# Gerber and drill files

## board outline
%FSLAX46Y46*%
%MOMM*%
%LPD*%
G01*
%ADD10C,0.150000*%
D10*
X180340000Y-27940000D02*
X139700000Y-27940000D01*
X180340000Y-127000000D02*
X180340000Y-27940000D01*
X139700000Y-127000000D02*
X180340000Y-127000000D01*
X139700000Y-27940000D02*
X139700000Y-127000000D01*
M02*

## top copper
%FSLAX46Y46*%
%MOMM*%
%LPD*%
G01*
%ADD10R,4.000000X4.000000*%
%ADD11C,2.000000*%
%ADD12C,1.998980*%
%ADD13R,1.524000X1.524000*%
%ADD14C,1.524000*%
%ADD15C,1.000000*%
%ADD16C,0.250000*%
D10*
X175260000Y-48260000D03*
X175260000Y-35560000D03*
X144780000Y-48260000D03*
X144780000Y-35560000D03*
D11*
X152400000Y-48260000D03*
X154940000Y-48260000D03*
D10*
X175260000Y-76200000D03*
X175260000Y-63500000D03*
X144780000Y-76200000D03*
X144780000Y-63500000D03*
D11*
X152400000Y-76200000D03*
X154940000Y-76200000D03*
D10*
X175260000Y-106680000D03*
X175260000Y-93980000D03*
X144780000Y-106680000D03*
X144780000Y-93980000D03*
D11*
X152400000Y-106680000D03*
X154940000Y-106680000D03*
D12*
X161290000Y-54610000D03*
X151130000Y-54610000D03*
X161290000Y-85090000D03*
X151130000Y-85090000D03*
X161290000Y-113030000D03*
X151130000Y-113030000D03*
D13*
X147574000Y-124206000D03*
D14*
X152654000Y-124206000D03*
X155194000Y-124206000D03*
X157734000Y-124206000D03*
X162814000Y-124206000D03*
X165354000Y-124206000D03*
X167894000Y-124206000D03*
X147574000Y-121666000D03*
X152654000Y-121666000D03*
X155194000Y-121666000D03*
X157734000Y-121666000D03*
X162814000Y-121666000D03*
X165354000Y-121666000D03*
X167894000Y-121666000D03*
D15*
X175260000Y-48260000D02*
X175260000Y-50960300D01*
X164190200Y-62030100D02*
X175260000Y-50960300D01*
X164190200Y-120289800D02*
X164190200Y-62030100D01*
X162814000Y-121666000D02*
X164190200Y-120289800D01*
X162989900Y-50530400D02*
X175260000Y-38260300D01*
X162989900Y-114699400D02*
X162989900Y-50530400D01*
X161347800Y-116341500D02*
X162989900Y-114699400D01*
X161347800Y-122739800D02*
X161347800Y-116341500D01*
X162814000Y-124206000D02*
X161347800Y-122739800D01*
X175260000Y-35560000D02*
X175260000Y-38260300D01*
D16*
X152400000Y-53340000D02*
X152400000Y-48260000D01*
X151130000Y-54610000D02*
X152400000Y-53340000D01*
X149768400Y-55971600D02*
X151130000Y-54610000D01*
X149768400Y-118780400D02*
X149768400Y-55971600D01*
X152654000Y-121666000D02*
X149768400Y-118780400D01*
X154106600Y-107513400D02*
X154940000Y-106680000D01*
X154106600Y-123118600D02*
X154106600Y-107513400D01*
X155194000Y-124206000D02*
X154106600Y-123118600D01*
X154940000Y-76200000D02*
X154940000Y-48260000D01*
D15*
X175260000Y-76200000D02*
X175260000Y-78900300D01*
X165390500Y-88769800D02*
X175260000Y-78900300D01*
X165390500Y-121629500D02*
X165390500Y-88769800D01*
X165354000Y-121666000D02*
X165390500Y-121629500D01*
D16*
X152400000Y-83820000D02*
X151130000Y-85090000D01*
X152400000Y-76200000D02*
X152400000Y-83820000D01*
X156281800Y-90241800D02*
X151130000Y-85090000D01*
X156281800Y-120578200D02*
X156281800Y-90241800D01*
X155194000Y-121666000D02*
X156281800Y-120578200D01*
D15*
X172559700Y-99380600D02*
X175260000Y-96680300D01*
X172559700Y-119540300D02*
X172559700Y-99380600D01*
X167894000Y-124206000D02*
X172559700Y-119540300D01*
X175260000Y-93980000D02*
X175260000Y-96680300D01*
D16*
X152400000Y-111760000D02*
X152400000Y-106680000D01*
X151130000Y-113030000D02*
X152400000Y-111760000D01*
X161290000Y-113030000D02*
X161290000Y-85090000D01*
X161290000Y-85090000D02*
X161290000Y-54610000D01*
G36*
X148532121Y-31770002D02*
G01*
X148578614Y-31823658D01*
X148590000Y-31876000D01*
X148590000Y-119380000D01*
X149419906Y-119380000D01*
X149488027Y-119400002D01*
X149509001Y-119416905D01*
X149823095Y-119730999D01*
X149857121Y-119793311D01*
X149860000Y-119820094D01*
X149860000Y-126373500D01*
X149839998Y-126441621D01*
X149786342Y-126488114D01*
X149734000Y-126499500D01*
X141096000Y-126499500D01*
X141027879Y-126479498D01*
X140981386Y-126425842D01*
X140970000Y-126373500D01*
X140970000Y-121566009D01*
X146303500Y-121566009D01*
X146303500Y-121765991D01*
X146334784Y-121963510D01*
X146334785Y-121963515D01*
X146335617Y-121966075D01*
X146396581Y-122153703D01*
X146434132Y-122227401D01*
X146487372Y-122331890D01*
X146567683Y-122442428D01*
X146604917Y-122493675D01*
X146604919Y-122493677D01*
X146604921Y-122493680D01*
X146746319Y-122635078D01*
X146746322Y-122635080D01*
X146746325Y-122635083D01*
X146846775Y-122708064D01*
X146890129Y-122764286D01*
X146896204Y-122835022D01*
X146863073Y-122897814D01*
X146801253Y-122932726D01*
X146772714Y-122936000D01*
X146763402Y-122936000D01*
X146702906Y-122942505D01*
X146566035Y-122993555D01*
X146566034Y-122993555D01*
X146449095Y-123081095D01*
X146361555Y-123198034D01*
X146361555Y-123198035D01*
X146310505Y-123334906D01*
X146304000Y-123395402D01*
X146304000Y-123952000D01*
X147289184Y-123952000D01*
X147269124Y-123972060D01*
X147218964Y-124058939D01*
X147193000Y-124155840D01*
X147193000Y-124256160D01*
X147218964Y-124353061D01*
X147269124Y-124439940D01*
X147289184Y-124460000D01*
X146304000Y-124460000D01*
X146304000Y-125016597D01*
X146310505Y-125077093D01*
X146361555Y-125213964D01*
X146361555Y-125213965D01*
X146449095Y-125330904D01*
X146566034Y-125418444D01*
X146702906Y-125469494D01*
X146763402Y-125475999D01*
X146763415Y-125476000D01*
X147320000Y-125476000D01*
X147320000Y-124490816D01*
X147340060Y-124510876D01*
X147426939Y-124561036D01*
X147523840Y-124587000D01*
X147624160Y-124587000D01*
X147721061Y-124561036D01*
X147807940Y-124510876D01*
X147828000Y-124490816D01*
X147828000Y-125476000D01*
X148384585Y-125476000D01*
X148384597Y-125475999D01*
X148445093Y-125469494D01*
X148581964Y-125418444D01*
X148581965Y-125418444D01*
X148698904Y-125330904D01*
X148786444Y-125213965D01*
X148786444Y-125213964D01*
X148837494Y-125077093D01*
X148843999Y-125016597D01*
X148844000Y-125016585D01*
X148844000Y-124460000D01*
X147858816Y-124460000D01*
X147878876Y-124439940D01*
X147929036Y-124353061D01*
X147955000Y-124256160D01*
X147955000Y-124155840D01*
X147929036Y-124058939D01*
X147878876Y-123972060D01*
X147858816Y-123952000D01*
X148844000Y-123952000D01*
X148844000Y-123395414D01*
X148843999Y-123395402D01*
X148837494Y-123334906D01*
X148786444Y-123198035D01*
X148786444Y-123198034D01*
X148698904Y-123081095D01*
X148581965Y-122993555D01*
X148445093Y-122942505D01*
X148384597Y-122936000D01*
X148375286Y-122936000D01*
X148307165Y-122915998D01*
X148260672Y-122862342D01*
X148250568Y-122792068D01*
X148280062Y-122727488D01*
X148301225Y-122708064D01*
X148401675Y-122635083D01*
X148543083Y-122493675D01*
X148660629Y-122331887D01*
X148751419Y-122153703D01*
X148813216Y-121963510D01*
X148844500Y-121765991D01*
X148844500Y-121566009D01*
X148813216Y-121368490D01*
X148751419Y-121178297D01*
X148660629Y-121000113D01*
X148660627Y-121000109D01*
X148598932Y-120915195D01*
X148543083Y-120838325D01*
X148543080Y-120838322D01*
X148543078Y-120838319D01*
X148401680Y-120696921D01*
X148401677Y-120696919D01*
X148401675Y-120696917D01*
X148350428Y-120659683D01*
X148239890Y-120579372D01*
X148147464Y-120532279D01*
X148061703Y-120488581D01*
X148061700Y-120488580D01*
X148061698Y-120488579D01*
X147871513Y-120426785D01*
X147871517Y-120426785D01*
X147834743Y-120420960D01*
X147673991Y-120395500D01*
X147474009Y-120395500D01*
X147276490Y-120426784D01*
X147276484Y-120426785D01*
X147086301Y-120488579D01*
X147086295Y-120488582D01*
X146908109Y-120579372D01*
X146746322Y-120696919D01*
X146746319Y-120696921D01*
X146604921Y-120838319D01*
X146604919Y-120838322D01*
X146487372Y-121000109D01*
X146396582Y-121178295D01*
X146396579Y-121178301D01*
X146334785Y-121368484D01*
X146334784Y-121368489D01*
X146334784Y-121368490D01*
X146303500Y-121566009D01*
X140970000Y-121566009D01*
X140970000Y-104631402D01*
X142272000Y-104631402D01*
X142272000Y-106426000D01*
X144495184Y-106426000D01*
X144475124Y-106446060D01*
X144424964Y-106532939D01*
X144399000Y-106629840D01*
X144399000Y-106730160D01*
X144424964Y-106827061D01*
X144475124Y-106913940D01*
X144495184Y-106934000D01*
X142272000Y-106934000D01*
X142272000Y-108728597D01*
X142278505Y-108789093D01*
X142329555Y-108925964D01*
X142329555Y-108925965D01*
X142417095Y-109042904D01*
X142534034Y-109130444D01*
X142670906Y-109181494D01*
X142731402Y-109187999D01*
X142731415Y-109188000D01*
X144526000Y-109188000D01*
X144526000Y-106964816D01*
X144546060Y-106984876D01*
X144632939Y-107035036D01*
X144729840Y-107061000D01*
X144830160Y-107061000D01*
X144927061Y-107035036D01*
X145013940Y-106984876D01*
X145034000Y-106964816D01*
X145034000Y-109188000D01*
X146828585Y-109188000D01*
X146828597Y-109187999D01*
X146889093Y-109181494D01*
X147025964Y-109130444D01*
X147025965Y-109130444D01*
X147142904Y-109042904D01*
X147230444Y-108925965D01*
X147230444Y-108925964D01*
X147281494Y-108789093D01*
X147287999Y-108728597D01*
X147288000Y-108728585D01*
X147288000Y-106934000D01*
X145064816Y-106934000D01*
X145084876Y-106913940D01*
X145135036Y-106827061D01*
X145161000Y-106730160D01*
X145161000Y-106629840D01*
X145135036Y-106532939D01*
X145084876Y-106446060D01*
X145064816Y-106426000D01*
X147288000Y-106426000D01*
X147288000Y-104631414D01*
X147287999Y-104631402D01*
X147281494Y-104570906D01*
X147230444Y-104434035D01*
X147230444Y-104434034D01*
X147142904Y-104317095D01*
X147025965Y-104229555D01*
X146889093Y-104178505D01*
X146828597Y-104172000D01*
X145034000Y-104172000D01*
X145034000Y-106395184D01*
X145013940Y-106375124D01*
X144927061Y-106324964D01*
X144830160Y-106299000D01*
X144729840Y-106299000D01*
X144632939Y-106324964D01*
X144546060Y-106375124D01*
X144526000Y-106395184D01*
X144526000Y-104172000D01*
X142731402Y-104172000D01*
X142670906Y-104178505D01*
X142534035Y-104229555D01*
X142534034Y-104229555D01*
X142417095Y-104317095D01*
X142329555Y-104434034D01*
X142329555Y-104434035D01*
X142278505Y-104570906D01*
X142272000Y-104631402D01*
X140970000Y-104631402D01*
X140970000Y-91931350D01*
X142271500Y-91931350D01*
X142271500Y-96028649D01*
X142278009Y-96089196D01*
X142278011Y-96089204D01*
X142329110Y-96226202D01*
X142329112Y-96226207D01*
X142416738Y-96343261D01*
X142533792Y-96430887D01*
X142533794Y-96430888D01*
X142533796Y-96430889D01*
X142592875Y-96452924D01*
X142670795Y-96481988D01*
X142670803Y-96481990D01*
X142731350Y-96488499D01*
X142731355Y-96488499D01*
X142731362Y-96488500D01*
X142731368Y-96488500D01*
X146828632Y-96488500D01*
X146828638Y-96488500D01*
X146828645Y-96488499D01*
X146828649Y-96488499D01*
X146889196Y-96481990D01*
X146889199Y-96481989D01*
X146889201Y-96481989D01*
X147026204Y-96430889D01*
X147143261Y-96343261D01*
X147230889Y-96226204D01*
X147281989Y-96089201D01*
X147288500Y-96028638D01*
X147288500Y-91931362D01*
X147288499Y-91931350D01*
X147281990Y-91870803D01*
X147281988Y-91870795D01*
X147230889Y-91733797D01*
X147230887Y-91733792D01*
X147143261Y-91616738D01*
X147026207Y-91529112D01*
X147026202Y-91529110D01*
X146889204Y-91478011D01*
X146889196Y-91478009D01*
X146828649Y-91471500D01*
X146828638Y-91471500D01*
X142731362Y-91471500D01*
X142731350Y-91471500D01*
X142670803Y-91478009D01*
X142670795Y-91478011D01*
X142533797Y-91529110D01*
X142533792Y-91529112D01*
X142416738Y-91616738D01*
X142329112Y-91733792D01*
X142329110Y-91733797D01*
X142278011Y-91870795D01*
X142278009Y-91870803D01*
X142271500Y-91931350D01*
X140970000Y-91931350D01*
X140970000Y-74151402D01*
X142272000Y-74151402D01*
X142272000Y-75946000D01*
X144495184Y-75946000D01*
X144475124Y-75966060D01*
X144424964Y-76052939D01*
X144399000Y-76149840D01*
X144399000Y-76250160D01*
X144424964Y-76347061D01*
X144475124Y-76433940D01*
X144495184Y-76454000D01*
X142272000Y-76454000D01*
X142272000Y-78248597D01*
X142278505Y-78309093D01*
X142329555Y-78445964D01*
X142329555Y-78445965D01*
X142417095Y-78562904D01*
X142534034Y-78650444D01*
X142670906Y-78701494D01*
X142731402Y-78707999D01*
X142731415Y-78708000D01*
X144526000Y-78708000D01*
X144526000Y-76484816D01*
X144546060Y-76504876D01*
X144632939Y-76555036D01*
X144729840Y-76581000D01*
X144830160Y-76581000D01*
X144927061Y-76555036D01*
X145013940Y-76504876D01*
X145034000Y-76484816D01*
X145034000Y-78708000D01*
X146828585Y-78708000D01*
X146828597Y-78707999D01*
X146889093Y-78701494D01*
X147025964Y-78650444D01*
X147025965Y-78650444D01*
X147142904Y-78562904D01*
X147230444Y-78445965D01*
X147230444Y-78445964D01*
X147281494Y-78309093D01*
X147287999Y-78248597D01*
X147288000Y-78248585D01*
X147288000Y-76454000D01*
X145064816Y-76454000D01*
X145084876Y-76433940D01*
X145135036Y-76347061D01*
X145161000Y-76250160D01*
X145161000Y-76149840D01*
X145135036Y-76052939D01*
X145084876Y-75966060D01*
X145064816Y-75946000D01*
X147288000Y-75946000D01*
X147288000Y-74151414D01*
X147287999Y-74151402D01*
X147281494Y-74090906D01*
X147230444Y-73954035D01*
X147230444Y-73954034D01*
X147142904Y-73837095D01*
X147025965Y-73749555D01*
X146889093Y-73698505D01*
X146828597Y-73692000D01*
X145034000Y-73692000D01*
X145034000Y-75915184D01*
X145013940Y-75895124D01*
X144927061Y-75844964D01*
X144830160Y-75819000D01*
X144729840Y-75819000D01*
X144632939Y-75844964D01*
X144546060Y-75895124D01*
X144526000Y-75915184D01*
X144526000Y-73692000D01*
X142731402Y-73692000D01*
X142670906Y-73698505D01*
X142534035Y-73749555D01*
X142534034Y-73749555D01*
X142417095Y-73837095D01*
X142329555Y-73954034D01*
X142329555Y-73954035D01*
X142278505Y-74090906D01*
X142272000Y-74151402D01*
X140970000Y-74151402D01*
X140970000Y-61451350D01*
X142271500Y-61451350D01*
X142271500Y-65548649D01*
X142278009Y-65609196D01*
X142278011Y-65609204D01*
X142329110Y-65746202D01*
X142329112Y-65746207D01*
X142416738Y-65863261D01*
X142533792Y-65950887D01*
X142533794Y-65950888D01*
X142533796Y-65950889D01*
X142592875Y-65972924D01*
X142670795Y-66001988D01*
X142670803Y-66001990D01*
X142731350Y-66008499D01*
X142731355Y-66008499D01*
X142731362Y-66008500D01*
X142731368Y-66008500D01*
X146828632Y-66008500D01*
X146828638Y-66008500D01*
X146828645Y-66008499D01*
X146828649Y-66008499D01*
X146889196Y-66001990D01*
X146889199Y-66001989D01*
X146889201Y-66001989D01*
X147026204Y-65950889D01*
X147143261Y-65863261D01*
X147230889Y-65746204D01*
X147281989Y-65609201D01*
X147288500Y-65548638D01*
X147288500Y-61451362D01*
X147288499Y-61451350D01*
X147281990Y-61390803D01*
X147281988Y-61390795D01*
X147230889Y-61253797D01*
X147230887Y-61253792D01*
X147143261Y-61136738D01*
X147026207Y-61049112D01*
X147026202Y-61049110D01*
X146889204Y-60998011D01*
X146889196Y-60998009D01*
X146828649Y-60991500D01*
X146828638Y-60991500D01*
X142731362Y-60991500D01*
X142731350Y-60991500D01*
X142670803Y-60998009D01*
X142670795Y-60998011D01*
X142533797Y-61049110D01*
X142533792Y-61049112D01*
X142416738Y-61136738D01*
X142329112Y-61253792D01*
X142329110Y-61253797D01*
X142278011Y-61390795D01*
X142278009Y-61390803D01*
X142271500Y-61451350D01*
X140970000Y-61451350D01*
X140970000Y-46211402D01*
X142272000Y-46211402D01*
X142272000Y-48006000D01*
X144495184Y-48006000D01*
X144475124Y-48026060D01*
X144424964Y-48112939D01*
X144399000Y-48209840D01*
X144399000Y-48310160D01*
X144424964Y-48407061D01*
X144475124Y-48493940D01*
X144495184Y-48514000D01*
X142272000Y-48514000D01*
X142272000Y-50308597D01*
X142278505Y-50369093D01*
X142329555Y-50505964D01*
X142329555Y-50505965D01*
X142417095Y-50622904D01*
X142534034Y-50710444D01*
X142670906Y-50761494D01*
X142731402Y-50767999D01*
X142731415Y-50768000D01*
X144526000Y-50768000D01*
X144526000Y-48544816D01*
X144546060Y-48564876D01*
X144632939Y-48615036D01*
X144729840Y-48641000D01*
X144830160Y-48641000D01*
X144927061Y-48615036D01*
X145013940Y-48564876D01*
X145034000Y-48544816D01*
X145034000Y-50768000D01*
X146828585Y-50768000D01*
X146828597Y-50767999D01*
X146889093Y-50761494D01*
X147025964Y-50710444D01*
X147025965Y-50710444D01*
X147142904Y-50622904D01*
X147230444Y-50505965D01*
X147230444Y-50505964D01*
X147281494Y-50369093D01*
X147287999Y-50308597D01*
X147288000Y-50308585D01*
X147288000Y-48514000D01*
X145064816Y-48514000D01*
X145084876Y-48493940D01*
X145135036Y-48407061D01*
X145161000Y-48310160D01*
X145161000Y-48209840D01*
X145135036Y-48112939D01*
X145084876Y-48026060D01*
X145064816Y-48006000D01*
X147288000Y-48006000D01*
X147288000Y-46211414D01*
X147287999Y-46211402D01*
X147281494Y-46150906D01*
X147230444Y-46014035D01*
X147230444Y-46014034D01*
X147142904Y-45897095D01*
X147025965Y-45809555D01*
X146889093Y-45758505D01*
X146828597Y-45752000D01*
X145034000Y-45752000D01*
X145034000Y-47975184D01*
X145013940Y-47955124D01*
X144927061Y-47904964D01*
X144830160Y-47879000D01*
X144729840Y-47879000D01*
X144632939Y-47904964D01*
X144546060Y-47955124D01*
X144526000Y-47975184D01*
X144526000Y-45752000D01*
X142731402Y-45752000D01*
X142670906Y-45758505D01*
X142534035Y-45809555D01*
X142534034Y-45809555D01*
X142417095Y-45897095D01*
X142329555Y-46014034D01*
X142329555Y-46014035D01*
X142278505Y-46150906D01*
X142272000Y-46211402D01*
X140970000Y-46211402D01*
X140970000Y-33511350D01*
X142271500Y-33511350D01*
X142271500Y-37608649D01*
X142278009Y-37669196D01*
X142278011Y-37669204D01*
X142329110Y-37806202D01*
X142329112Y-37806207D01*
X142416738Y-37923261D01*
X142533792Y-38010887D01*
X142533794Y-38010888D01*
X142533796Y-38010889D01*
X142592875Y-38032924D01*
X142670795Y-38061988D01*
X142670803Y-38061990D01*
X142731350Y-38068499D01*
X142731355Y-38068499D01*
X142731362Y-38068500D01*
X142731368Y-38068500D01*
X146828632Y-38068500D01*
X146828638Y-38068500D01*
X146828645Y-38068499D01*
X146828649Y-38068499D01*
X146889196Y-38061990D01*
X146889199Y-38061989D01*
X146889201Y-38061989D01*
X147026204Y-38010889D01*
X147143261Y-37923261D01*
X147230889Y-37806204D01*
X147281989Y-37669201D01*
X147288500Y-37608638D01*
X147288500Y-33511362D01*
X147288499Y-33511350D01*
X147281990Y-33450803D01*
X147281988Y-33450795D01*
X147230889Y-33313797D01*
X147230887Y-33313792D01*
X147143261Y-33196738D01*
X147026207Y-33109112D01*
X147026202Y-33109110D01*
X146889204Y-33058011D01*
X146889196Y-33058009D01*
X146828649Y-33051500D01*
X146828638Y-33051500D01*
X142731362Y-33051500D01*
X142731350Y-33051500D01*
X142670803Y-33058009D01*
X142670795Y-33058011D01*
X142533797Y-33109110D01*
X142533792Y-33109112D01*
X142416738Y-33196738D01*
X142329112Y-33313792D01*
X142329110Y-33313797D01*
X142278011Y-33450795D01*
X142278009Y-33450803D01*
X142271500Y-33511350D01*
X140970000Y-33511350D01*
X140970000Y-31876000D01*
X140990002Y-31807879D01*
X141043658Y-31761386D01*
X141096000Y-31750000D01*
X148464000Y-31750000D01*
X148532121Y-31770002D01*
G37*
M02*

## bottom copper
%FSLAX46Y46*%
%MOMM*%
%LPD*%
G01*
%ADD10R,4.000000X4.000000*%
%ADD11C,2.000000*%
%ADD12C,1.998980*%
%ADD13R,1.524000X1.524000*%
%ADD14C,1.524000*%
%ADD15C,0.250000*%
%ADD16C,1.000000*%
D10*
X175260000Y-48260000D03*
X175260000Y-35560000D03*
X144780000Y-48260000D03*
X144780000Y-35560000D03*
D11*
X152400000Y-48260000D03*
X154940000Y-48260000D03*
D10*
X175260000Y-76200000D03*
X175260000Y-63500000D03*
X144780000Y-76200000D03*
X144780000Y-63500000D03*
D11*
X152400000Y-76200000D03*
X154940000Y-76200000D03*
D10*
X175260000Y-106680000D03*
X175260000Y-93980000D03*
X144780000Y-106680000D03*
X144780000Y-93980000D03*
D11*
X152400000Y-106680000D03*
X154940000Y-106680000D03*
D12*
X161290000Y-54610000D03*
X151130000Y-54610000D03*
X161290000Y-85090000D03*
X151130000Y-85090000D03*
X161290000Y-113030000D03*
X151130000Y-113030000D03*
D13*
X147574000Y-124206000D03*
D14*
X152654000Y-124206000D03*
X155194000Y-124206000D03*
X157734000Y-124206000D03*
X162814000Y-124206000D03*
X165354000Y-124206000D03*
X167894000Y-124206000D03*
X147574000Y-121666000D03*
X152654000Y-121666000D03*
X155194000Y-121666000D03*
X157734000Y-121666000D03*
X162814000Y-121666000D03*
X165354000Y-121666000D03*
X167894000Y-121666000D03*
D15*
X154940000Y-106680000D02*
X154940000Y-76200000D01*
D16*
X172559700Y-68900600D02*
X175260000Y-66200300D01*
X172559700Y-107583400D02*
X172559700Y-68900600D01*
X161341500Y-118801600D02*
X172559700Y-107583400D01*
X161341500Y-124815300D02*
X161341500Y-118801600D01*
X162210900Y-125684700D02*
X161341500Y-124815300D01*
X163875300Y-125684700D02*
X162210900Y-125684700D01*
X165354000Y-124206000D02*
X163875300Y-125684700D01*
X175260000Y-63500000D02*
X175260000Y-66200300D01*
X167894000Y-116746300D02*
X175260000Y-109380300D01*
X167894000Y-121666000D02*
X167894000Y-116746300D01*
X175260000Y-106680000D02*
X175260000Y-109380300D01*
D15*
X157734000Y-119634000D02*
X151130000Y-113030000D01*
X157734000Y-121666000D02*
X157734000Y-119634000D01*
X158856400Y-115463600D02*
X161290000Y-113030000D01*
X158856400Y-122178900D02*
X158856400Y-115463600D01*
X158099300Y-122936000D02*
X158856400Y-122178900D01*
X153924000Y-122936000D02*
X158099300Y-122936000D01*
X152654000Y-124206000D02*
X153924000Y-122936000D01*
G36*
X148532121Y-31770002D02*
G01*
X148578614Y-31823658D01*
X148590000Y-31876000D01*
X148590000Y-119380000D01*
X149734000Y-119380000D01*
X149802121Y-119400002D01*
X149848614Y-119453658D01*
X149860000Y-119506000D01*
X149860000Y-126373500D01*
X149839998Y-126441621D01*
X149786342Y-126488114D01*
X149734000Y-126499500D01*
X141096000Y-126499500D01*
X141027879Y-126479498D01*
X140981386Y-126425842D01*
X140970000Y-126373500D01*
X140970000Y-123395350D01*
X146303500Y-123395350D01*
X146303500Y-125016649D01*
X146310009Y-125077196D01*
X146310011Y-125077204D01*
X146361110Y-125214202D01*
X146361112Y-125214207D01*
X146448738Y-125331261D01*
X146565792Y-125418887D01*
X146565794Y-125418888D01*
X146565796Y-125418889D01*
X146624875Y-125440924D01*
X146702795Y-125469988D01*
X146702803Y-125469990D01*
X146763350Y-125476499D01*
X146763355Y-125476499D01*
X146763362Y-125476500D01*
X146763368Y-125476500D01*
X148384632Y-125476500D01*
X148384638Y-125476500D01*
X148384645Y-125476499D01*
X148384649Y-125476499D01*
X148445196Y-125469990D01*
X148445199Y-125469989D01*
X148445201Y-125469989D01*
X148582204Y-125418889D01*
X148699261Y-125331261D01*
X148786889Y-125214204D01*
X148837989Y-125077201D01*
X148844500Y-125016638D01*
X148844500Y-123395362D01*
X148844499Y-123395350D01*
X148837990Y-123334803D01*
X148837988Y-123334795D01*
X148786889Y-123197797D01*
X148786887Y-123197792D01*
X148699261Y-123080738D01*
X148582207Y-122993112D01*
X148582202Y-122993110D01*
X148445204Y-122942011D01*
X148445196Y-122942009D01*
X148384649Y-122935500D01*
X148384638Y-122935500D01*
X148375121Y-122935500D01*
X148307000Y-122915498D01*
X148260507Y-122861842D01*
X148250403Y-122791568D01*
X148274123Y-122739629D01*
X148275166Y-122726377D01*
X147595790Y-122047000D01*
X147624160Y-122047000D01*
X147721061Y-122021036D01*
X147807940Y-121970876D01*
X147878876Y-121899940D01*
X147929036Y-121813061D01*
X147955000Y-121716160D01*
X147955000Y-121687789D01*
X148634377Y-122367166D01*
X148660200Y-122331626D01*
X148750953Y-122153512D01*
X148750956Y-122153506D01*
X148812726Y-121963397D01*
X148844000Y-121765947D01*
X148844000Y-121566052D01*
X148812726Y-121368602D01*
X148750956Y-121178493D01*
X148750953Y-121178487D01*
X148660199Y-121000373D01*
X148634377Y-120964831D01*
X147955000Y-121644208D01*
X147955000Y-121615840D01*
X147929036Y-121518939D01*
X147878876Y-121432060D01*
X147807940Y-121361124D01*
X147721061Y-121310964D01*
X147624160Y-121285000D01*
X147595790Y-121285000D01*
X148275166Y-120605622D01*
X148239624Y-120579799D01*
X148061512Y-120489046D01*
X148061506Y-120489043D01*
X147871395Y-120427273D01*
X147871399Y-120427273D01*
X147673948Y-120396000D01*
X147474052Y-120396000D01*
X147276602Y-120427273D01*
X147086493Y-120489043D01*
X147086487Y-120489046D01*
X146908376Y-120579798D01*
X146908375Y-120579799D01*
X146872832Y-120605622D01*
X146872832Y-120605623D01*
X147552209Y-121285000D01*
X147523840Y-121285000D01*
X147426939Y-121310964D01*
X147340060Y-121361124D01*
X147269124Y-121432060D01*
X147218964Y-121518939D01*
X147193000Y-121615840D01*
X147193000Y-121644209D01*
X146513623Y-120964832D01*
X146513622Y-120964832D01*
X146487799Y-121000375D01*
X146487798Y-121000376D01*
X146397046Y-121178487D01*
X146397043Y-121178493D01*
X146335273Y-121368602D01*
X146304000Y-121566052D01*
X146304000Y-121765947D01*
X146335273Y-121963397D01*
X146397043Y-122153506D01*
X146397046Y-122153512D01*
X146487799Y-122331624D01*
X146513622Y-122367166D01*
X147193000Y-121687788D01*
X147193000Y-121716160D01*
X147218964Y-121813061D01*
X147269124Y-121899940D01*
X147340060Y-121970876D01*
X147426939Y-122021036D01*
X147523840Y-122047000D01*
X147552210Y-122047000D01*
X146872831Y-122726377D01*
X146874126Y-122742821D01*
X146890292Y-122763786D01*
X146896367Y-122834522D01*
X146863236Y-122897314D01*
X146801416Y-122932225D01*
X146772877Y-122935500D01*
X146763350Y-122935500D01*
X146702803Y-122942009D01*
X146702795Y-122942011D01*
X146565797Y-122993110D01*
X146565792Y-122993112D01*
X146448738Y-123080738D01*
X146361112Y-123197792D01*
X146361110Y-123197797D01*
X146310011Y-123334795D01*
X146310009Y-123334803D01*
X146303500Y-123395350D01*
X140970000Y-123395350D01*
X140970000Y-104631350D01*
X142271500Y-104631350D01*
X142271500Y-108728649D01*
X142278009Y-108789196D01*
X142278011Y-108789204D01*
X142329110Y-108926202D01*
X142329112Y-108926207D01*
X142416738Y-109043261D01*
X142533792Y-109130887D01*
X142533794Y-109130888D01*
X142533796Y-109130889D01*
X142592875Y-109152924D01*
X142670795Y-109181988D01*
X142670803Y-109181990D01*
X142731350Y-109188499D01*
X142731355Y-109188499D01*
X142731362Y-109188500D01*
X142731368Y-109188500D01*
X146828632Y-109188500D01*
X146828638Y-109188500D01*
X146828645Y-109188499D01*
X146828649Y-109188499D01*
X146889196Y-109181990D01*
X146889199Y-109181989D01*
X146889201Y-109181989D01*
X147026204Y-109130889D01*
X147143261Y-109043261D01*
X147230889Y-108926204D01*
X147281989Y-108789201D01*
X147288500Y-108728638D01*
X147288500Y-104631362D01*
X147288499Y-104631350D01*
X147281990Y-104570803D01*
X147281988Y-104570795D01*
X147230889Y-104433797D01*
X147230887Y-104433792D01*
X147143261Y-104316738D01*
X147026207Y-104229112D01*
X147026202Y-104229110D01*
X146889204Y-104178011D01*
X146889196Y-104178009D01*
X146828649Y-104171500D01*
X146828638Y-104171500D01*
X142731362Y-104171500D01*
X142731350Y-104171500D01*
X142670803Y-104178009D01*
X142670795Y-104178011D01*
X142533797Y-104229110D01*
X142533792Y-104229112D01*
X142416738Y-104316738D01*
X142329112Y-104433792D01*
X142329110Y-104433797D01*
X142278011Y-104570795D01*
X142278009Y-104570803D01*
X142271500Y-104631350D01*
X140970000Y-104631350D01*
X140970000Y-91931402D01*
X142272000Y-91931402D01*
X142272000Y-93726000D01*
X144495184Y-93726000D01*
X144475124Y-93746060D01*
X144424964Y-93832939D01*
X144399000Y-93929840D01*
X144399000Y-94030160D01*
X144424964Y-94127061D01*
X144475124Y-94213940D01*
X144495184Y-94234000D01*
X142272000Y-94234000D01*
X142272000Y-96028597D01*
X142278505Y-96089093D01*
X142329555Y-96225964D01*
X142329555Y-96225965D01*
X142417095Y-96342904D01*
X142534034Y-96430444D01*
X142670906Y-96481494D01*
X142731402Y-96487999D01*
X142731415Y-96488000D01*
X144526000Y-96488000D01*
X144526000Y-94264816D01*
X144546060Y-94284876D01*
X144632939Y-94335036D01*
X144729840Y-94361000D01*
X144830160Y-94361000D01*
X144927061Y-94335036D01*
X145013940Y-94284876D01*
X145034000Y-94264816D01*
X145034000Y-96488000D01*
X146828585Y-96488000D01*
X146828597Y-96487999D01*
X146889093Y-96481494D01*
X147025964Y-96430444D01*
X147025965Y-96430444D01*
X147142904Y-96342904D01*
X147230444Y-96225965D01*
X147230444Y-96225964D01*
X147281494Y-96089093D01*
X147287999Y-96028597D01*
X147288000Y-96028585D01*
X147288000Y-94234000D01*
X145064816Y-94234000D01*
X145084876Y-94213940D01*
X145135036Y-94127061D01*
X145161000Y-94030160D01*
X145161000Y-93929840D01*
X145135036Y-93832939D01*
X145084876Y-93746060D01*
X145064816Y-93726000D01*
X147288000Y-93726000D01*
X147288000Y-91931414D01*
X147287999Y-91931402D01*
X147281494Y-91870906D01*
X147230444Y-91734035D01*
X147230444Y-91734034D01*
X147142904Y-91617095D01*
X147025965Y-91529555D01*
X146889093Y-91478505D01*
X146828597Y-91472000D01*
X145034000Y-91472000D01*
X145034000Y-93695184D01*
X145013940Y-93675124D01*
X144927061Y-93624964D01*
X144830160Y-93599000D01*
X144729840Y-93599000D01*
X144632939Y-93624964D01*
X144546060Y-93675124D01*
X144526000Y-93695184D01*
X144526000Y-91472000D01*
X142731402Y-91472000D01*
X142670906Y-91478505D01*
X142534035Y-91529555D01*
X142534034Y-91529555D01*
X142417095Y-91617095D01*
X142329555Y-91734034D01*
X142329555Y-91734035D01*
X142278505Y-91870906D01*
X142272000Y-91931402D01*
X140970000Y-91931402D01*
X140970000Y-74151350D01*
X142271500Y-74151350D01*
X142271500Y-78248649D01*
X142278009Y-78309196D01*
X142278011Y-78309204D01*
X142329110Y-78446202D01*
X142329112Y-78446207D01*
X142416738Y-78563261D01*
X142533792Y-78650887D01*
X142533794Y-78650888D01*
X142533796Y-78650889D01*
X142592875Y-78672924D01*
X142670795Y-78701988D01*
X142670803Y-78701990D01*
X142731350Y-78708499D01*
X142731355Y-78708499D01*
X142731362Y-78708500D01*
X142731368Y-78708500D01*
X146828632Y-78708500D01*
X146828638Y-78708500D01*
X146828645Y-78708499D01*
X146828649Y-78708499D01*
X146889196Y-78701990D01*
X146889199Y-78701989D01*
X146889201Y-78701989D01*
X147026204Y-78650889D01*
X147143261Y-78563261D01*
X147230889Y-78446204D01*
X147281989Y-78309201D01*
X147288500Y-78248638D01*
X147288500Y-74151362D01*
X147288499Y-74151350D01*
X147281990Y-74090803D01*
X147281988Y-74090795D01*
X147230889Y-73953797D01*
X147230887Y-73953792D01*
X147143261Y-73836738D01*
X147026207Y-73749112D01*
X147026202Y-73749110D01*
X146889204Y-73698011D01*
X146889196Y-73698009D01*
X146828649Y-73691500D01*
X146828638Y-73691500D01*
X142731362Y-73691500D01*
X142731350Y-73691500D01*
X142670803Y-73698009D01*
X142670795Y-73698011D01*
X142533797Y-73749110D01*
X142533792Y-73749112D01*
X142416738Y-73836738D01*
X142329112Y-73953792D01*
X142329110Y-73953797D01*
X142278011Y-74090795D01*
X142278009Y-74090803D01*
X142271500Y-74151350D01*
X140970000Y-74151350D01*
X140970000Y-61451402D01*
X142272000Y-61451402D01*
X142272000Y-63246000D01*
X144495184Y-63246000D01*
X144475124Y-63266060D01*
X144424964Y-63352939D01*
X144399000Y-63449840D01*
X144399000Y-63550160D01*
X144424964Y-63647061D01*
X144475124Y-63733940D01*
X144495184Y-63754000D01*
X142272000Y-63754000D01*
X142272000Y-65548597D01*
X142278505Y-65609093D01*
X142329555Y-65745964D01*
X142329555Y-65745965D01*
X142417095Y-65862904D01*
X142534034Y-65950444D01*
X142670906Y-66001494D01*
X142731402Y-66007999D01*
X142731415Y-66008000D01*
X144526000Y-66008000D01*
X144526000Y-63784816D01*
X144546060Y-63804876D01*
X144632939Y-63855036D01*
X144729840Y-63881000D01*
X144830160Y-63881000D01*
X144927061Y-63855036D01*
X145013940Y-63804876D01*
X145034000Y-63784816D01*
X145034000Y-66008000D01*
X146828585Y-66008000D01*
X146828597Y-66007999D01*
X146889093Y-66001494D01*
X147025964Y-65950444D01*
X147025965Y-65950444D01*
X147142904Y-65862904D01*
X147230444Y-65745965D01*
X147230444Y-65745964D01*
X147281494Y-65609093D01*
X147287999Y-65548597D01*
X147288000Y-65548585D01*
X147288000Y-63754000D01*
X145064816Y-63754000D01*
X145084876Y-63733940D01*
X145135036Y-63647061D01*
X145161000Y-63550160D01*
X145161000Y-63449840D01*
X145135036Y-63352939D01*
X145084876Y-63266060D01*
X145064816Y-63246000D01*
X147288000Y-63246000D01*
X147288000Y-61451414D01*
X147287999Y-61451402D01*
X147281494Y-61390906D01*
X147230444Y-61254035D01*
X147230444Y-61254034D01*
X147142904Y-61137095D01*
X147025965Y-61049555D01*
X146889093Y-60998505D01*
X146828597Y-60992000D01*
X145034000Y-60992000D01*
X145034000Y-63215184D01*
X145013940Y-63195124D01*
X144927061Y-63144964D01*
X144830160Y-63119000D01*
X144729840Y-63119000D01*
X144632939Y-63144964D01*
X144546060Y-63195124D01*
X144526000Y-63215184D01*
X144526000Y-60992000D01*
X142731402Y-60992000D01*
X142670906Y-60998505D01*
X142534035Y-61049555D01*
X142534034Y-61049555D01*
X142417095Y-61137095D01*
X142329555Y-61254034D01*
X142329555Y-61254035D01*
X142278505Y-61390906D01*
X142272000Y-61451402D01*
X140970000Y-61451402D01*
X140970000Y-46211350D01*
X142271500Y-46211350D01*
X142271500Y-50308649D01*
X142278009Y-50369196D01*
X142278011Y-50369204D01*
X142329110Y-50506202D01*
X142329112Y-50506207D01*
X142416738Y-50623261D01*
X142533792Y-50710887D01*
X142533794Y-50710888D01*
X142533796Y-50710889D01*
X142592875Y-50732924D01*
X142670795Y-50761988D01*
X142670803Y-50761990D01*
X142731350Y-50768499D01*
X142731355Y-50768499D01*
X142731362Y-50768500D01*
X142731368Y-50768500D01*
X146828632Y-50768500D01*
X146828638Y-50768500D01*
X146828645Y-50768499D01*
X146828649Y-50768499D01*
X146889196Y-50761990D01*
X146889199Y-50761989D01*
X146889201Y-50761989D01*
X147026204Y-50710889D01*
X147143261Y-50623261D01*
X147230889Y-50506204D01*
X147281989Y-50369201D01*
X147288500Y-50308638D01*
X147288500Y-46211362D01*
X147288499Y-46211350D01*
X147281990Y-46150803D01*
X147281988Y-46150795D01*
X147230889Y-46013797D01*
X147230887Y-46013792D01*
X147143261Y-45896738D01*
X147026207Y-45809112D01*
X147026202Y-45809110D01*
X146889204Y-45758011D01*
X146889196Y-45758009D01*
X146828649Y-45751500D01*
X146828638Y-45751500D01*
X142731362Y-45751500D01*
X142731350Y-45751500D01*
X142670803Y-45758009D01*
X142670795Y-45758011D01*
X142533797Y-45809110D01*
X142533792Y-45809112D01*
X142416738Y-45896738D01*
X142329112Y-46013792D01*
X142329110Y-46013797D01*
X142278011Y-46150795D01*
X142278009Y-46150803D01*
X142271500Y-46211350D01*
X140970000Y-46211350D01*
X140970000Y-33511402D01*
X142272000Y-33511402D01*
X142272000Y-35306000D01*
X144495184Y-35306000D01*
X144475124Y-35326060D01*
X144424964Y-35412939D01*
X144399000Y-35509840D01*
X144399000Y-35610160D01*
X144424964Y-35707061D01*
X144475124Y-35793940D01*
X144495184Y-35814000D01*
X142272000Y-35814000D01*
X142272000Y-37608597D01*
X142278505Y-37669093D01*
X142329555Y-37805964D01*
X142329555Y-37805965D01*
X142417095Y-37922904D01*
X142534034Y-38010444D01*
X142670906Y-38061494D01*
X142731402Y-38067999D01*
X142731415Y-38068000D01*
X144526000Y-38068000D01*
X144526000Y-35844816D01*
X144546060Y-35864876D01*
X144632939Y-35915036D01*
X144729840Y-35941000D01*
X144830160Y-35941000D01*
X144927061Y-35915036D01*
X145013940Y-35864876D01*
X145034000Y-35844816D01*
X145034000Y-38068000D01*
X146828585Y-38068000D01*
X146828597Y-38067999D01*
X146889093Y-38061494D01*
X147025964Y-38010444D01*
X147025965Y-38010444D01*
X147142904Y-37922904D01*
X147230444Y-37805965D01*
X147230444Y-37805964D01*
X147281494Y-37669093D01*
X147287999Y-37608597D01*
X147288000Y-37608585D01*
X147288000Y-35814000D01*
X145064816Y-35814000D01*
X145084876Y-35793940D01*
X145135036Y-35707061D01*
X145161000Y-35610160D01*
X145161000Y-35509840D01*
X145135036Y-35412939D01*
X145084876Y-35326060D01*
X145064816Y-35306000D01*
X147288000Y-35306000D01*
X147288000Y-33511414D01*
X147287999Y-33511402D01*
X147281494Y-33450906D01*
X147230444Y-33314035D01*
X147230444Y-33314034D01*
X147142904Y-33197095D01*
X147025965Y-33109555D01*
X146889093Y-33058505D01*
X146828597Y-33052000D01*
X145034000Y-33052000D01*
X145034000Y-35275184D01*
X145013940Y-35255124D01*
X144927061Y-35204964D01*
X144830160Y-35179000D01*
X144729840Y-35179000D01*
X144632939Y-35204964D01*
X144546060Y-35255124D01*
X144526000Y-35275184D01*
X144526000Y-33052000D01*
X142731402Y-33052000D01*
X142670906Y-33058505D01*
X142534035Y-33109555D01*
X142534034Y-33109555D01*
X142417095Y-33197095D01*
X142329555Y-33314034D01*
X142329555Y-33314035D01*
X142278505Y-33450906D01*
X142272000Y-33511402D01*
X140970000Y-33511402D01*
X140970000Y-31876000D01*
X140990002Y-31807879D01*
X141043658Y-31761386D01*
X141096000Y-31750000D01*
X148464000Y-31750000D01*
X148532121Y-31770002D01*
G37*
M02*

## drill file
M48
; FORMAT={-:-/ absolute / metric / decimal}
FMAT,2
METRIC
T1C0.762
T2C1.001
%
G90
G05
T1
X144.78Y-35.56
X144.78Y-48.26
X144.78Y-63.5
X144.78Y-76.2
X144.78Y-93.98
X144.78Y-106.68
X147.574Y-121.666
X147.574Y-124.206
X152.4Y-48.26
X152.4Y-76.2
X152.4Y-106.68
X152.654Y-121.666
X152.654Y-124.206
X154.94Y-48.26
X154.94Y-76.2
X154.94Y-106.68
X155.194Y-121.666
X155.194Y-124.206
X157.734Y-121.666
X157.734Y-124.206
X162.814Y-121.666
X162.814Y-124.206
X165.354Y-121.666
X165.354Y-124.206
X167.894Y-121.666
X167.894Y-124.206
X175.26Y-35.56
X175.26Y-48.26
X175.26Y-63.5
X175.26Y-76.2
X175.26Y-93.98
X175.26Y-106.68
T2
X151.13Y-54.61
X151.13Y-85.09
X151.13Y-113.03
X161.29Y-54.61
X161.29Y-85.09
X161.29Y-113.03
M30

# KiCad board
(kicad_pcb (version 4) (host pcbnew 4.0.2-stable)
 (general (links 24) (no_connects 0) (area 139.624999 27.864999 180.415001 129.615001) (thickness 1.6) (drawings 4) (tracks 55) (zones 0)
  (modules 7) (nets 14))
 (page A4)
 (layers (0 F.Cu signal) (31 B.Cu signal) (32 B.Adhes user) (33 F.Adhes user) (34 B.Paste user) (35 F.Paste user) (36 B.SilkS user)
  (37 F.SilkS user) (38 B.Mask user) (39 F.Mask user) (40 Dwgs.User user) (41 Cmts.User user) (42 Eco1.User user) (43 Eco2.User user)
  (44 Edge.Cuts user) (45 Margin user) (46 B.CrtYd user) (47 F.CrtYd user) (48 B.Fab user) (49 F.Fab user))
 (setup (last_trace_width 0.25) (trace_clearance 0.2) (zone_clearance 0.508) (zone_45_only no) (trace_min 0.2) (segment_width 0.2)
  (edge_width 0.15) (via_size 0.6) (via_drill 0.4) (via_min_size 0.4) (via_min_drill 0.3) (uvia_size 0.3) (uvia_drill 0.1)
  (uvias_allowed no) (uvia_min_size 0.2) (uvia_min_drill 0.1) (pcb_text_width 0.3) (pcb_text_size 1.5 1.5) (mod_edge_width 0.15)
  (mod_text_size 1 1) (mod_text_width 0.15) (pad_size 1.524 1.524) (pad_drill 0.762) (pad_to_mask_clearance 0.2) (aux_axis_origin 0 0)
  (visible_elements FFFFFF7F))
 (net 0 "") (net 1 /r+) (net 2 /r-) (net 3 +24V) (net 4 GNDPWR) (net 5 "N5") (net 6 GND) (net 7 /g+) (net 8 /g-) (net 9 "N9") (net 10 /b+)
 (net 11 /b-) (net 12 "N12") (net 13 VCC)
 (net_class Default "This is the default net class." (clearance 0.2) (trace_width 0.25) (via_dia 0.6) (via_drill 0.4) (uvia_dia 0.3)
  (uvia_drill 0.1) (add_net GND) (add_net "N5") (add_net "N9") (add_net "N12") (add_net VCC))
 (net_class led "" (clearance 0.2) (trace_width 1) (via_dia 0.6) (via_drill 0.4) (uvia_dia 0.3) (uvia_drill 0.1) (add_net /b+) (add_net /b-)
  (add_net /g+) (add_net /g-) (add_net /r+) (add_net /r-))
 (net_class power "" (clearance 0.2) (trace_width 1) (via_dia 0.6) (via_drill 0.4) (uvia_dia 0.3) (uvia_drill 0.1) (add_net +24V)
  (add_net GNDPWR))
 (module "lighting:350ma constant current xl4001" (layer F.Cu) (at 175.26 48.26 90)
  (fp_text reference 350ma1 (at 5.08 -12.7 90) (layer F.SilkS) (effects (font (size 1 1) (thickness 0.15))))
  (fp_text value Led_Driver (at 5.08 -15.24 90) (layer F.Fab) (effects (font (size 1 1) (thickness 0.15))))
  (pad 3 thru_hole rect (at 0 0 90) (size 4 4) (drill 0.762) (layers *.Cu *.Mask F.SilkS) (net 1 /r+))
  (pad 4 thru_hole rect (at 12.7 0 90) (size 4 4) (drill 0.762) (layers *.Cu *.Mask F.SilkS) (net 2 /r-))
  (pad 1 thru_hole rect (at 0 -30.48 90) (size 4 4) (drill 0.762) (layers *.Cu *.Mask F.SilkS) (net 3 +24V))
  (pad 2 thru_hole rect (at 12.7 -30.48 90) (size 4 4) (drill 0.762) (layers *.Cu *.Mask F.SilkS) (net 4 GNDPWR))
  (pad 5 thru_hole circle (at 0 -22.86 90) (size 2 2) (drill 0.762) (layers *.Cu *.Mask F.SilkS) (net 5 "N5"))
  (pad 6 thru_hole circle (at 0 -20.32 90) (size 2 2) (drill 0.762) (layers *.Cu *.Mask F.SilkS) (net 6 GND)))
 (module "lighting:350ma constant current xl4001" (layer F.Cu) (at 175.26 76.2 90)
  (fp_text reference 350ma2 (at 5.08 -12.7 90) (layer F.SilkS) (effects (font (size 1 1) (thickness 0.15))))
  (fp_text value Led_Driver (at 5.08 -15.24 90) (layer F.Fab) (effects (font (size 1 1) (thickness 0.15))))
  (pad 3 thru_hole rect (at 0 0 90) (size 4 4) (drill 0.762) (layers *.Cu *.Mask F.SilkS) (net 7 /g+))
  (pad 4 thru_hole rect (at 12.7 0 90) (size 4 4) (drill 0.762) (layers *.Cu *.Mask F.SilkS) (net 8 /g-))
  (pad 1 thru_hole rect (at 0 -30.48 90) (size 4 4) (drill 0.762) (layers *.Cu *.Mask F.SilkS) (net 3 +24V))
  (pad 2 thru_hole rect (at 12.7 -30.48 90) (size 4 4) (drill 0.762) (layers *.Cu *.Mask F.SilkS) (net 4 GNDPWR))
  (pad 5 thru_hole circle (at 0 -22.86 90) (size 2 2) (drill 0.762) (layers *.Cu *.Mask F.SilkS) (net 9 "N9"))
  (pad 6 thru_hole circle (at 0 -20.32 90) (size 2 2) (drill 0.762) (layers *.Cu *.Mask F.SilkS) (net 6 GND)))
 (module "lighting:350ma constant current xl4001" (layer F.Cu) (at 175.26 106.68 90)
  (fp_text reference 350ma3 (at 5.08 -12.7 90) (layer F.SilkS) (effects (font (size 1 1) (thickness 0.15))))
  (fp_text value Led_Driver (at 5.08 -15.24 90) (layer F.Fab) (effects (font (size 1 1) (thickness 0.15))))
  (pad 3 thru_hole rect (at 0 0 90) (size 4 4) (drill 0.762) (layers *.Cu *.Mask F.SilkS) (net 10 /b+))
  (pad 4 thru_hole rect (at 12.7 0 90) (size 4 4) (drill 0.762) (layers *.Cu *.Mask F.SilkS) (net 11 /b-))
  (pad 1 thru_hole rect (at 0 -30.48 90) (size 4 4) (drill 0.762) (layers *.Cu *.Mask F.SilkS) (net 3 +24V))
  (pad 2 thru_hole rect (at 12.7 -30.48 90) (size 4 4) (drill 0.762) (layers *.Cu *.Mask F.SilkS) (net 4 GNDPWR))
  (pad 5 thru_hole circle (at 0 -22.86 90) (size 2 2) (drill 0.762) (layers *.Cu *.Mask F.SilkS) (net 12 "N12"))
  (pad 6 thru_hole circle (at 0 -20.32 90) (size 2 2) (drill 0.762) (layers *.Cu *.Mask F.SilkS) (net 6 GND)))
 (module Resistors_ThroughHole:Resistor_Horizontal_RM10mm (layer F.Cu) (at 161.29 54.61 180)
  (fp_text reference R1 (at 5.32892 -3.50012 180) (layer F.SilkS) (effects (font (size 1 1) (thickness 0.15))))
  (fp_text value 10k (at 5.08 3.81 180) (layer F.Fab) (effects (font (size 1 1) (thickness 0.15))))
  (pad 1 thru_hole circle (at 0 0 180) (size 1.99898 1.99898) (drill 1.00076) (layers *.Cu *.SilkS *.Mask) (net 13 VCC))
  (pad 2 thru_hole circle (at 10.16 0 180) (size 1.99898 1.99898) (drill 1.00076) (layers *.Cu *.SilkS *.Mask) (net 5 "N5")))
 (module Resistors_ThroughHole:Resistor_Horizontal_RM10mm (layer F.Cu) (at 161.29 85.09 180)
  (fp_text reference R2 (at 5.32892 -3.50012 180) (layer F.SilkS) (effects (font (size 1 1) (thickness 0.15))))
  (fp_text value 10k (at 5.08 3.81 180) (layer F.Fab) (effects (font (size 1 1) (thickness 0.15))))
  (pad 1 thru_hole circle (at 0 0 180) (size 1.99898 1.99898) (drill 1.00076) (layers *.Cu *.SilkS *.Mask) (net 13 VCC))
  (pad 2 thru_hole circle (at 10.16 0 180) (size 1.99898 1.99898) (drill 1.00076) (layers *.Cu *.SilkS *.Mask) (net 9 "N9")))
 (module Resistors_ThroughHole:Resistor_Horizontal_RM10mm (layer F.Cu) (at 161.29 113.03 180)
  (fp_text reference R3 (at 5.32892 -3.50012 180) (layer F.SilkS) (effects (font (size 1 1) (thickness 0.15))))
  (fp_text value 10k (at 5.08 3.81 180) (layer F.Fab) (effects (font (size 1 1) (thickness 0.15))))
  (pad 1 thru_hole circle (at 0 0 180) (size 1.99898 1.99898) (drill 1.00076) (layers *.Cu *.SilkS *.Mask) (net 13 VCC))
  (pad 2 thru_hole circle (at 10.16 0 180) (size 1.99898 1.99898) (drill 1.00076) (layers *.Cu *.SilkS *.Mask) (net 12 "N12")))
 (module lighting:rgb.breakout (layer F.Cu) (at 150.114 124.206)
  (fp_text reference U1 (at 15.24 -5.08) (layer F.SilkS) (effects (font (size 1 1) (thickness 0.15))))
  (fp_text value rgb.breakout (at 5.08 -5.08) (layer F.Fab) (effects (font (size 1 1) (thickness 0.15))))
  (pad 1 thru_hole rect (at -2.54 0) (size 1.524 1.524) (drill 0.762) (layers *.Cu *.Mask F.SilkS) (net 3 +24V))
  (pad 3 thru_hole circle (at 2.54 0) (size 1.524 1.524) (drill 0.762) (layers *.Cu *.Mask F.SilkS) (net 13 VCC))
  (pad 4 thru_hole circle (at 5.08 0) (size 1.524 1.524) (drill 0.762) (layers *.Cu *.Mask F.SilkS) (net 6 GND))
  (pad "" thru_hole circle (at 7.62 0) (size 1.524 1.524) (drill 0.762) (layers *.Cu *.Mask F.SilkS))
  (pad 9 thru_hole circle (at 12.7 0) (size 1.524 1.524) (drill 0.762) (layers *.Cu *.Mask F.SilkS) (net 2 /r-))
  (pad 11 thru_hole circle (at 15.24 0) (size 1.524 1.524) (drill 0.762) (layers *.Cu *.Mask F.SilkS) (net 8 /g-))
  (pad 13 thru_hole circle (at 17.78 0) (size 1.524 1.524) (drill 0.762) (layers *.Cu *.Mask F.SilkS) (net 11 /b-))
  (pad 2 thru_hole circle (at -2.54 -2.54) (size 1.524 1.524) (drill 0.762) (layers *.Cu *.Mask F.SilkS) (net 4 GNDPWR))
  (pad 5 thru_hole circle (at 2.54 -2.54) (size 1.524 1.524) (drill 0.762) (layers *.Cu *.Mask F.SilkS) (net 5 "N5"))
  (pad 6 thru_hole circle (at 5.08 -2.54) (size 1.524 1.524) (drill 0.762) (layers *.Cu *.Mask F.SilkS) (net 9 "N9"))
  (pad 7 thru_hole circle (at 7.62 -2.54) (size 1.524 1.524) (drill 0.762) (layers *.Cu *.Mask F.SilkS) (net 12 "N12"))
  (pad 8 thru_hole circle (at 12.7 -2.54) (size 1.524 1.524) (drill 0.762) (layers *.Cu *.Mask F.SilkS) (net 1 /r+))
  (pad 10 thru_hole circle (at 15.24 -2.54) (size 1.524 1.524) (drill 0.762) (layers *.Cu *.Mask F.SilkS) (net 7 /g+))
  (pad 12 thru_hole circle (at 17.78 -2.54) (size 1.524 1.524) (drill 0.762) (layers *.Cu *.Mask F.SilkS) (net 10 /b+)))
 (gr_line (start 180.34 27.94) (end 139.7 27.94) (angle 90) (layer Edge.Cuts) (width 0.15))
 (gr_line (start 180.34 127) (end 180.34 27.94) (angle 90) (layer Edge.Cuts) (width 0.15))
 (gr_line (start 139.7 127) (end 180.34 127) (angle 90) (layer Edge.Cuts) (width 0.15))
 (gr_line (start 139.7 27.94) (end 139.7 127) (angle 90) (layer Edge.Cuts) (width 0.15))
 (segment (start 175.26 48.26) (end 175.26 50.9603) (width 1) (layer F.Cu) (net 1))
 (segment (start 164.1902 62.0301) (end 175.26 50.9603) (width 1) (layer F.Cu) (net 1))
 (segment (start 164.1902 120.2898) (end 164.1902 62.0301) (width 1) (layer F.Cu) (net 1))
 (segment (start 162.814 121.666) (end 164.1902 120.2898) (width 1) (layer F.Cu) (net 1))
 (segment (start 162.9899 50.5304) (end 175.26 38.2603) (width 1) (layer F.Cu) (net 2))
 (segment (start 162.9899 114.6994) (end 162.9899 50.5304) (width 1) (layer F.Cu) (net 2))
 (segment (start 161.3478 116.3415) (end 162.9899 114.6994) (width 1) (layer F.Cu) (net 2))
 (segment (start 161.3478 122.7398) (end 161.3478 116.3415) (width 1) (layer F.Cu) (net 2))
 (segment (start 162.814 124.206) (end 161.3478 122.7398) (width 1) (layer F.Cu) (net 2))
 (segment (start 175.26 35.56) (end 175.26 38.2603) (width 1) (layer F.Cu) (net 2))
 (segment (start 152.4 53.34) (end 152.4 48.26) (width 0.25) (layer F.Cu) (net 5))
 (segment (start 151.13 54.61) (end 152.4 53.34) (width 0.25) (layer F.Cu) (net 5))
 (segment (start 149.7684 55.9716) (end 151.13 54.61) (width 0.25) (layer F.Cu) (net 5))
 (segment (start 149.7684 118.7804) (end 149.7684 55.9716) (width 0.25) (layer F.Cu) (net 5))
 (segment (start 152.654 121.666) (end 149.7684 118.7804) (width 0.25) (layer F.Cu) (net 5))
 (segment (start 154.1066 107.5134) (end 154.94 106.68) (width 0.25) (layer F.Cu) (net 6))
 (segment (start 154.1066 123.1186) (end 154.1066 107.5134) (width 0.25) (layer F.Cu) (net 6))
 (segment (start 155.194 124.206) (end 154.1066 123.1186) (width 0.25) (layer F.Cu) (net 6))
 (segment (start 154.94 106.68) (end 154.94 76.2) (width 0.25) (layer B.Cu) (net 6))
 (segment (start 154.94 76.2) (end 154.94 48.26) (width 0.25) (layer F.Cu) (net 6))
 (segment (start 175.26 76.2) (end 175.26 78.9003) (width 1) (layer F.Cu) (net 7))
 (segment (start 165.3905 88.7698) (end 175.26 78.9003) (width 1) (layer F.Cu) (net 7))
 (segment (start 165.3905 121.6295) (end 165.3905 88.7698) (width 1) (layer F.Cu) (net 7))
 (segment (start 165.354 121.666) (end 165.3905 121.6295) (width 1) (layer F.Cu) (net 7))
 (segment (start 172.5597 68.9006) (end 175.26 66.2003) (width 1) (layer B.Cu) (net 8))
 (segment (start 172.5597 107.5834) (end 172.5597 68.9006) (width 1) (layer B.Cu) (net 8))
 (segment (start 161.3415 118.8016) (end 172.5597 107.5834) (width 1) (layer B.Cu) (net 8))
 (segment (start 161.3415 124.8153) (end 161.3415 118.8016) (width 1) (layer B.Cu) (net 8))
 (segment (start 162.2109 125.6847) (end 161.3415 124.8153) (width 1) (layer B.Cu) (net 8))
 (segment (start 163.8753 125.6847) (end 162.2109 125.6847) (width 1) (layer B.Cu) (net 8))
 (segment (start 165.354 124.206) (end 163.8753 125.6847) (width 1) (layer B.Cu) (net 8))
 (segment (start 175.26 63.5) (end 175.26 66.2003) (width 1) (layer B.Cu) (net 8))
 (segment (start 152.4 83.82) (end 151.13 85.09) (width 0.25) (layer F.Cu) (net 9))
 (segment (start 152.4 76.2) (end 152.4 83.82) (width 0.25) (layer F.Cu) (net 9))
 (segment (start 156.2818 90.2418) (end 151.13 85.09) (width 0.25) (layer F.Cu) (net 9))
 (segment (start 156.2818 120.5782) (end 156.2818 90.2418) (width 0.25) (layer F.Cu) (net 9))
 (segment (start 155.194 121.666) (end 156.2818 120.5782) (width 0.25) (layer F.Cu) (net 9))
 (segment (start 167.894 116.7463) (end 175.26 109.3803) (width 1) (layer B.Cu) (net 10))
 (segment (start 167.894 121.666) (end 167.894 116.7463) (width 1) (layer B.Cu) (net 10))
 (segment (start 175.26 106.68) (end 175.26 109.3803) (width 1) (layer B.Cu) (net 10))
 (segment (start 172.5597 99.3806) (end 175.26 96.6803) (width 1) (layer F.Cu) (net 11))
 (segment (start 172.5597 119.5403) (end 172.5597 99.3806) (width 1) (layer F.Cu) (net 11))
 (segment (start 167.894 124.206) (end 172.5597 119.5403) (width 1) (layer F.Cu) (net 11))
 (segment (start 175.26 93.98) (end 175.26 96.6803) (width 1) (layer F.Cu) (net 11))
 (segment (start 157.734 119.634) (end 151.13 113.03) (width 0.25) (layer B.Cu) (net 12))
 (segment (start 157.734 121.666) (end 157.734 119.634) (width 0.25) (layer B.Cu) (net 12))
 (segment (start 152.4 111.76) (end 152.4 106.68) (width 0.25) (layer F.Cu) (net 12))
 (segment (start 151.13 113.03) (end 152.4 111.76) (width 0.25) (layer F.Cu) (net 12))
 (segment (start 158.8564 115.4636) (end 161.29 113.03) (width 0.25) (layer B.Cu) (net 13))
 (segment (start 158.8564 122.1789) (end 158.8564 115.4636) (width 0.25) (layer B.Cu) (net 13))
 (segment (start 158.0993 122.936) (end 158.8564 122.1789) (width 0.25) (layer B.Cu) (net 13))
 (segment (start 153.924 122.936) (end 158.0993 122.936) (width 0.25) (layer B.Cu) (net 13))
 (segment (start 152.654 124.206) (end 153.924 122.936) (width 0.25) (layer B.Cu) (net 13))
 (segment (start 161.29 113.03) (end 161.29 85.09) (width 0.25) (layer F.Cu) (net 13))
 (segment (start 161.29 85.09) (end 161.29 54.61) (width 0.25) (layer F.Cu) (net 13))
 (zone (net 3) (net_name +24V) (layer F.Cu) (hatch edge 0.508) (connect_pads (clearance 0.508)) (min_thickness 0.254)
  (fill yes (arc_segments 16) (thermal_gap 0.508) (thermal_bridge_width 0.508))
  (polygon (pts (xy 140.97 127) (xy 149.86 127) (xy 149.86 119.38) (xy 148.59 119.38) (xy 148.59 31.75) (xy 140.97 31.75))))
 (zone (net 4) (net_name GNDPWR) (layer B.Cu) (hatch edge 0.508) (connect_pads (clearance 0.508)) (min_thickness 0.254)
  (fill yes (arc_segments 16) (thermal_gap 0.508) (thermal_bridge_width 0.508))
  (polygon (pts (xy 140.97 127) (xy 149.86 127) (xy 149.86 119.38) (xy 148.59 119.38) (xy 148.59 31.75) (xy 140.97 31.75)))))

